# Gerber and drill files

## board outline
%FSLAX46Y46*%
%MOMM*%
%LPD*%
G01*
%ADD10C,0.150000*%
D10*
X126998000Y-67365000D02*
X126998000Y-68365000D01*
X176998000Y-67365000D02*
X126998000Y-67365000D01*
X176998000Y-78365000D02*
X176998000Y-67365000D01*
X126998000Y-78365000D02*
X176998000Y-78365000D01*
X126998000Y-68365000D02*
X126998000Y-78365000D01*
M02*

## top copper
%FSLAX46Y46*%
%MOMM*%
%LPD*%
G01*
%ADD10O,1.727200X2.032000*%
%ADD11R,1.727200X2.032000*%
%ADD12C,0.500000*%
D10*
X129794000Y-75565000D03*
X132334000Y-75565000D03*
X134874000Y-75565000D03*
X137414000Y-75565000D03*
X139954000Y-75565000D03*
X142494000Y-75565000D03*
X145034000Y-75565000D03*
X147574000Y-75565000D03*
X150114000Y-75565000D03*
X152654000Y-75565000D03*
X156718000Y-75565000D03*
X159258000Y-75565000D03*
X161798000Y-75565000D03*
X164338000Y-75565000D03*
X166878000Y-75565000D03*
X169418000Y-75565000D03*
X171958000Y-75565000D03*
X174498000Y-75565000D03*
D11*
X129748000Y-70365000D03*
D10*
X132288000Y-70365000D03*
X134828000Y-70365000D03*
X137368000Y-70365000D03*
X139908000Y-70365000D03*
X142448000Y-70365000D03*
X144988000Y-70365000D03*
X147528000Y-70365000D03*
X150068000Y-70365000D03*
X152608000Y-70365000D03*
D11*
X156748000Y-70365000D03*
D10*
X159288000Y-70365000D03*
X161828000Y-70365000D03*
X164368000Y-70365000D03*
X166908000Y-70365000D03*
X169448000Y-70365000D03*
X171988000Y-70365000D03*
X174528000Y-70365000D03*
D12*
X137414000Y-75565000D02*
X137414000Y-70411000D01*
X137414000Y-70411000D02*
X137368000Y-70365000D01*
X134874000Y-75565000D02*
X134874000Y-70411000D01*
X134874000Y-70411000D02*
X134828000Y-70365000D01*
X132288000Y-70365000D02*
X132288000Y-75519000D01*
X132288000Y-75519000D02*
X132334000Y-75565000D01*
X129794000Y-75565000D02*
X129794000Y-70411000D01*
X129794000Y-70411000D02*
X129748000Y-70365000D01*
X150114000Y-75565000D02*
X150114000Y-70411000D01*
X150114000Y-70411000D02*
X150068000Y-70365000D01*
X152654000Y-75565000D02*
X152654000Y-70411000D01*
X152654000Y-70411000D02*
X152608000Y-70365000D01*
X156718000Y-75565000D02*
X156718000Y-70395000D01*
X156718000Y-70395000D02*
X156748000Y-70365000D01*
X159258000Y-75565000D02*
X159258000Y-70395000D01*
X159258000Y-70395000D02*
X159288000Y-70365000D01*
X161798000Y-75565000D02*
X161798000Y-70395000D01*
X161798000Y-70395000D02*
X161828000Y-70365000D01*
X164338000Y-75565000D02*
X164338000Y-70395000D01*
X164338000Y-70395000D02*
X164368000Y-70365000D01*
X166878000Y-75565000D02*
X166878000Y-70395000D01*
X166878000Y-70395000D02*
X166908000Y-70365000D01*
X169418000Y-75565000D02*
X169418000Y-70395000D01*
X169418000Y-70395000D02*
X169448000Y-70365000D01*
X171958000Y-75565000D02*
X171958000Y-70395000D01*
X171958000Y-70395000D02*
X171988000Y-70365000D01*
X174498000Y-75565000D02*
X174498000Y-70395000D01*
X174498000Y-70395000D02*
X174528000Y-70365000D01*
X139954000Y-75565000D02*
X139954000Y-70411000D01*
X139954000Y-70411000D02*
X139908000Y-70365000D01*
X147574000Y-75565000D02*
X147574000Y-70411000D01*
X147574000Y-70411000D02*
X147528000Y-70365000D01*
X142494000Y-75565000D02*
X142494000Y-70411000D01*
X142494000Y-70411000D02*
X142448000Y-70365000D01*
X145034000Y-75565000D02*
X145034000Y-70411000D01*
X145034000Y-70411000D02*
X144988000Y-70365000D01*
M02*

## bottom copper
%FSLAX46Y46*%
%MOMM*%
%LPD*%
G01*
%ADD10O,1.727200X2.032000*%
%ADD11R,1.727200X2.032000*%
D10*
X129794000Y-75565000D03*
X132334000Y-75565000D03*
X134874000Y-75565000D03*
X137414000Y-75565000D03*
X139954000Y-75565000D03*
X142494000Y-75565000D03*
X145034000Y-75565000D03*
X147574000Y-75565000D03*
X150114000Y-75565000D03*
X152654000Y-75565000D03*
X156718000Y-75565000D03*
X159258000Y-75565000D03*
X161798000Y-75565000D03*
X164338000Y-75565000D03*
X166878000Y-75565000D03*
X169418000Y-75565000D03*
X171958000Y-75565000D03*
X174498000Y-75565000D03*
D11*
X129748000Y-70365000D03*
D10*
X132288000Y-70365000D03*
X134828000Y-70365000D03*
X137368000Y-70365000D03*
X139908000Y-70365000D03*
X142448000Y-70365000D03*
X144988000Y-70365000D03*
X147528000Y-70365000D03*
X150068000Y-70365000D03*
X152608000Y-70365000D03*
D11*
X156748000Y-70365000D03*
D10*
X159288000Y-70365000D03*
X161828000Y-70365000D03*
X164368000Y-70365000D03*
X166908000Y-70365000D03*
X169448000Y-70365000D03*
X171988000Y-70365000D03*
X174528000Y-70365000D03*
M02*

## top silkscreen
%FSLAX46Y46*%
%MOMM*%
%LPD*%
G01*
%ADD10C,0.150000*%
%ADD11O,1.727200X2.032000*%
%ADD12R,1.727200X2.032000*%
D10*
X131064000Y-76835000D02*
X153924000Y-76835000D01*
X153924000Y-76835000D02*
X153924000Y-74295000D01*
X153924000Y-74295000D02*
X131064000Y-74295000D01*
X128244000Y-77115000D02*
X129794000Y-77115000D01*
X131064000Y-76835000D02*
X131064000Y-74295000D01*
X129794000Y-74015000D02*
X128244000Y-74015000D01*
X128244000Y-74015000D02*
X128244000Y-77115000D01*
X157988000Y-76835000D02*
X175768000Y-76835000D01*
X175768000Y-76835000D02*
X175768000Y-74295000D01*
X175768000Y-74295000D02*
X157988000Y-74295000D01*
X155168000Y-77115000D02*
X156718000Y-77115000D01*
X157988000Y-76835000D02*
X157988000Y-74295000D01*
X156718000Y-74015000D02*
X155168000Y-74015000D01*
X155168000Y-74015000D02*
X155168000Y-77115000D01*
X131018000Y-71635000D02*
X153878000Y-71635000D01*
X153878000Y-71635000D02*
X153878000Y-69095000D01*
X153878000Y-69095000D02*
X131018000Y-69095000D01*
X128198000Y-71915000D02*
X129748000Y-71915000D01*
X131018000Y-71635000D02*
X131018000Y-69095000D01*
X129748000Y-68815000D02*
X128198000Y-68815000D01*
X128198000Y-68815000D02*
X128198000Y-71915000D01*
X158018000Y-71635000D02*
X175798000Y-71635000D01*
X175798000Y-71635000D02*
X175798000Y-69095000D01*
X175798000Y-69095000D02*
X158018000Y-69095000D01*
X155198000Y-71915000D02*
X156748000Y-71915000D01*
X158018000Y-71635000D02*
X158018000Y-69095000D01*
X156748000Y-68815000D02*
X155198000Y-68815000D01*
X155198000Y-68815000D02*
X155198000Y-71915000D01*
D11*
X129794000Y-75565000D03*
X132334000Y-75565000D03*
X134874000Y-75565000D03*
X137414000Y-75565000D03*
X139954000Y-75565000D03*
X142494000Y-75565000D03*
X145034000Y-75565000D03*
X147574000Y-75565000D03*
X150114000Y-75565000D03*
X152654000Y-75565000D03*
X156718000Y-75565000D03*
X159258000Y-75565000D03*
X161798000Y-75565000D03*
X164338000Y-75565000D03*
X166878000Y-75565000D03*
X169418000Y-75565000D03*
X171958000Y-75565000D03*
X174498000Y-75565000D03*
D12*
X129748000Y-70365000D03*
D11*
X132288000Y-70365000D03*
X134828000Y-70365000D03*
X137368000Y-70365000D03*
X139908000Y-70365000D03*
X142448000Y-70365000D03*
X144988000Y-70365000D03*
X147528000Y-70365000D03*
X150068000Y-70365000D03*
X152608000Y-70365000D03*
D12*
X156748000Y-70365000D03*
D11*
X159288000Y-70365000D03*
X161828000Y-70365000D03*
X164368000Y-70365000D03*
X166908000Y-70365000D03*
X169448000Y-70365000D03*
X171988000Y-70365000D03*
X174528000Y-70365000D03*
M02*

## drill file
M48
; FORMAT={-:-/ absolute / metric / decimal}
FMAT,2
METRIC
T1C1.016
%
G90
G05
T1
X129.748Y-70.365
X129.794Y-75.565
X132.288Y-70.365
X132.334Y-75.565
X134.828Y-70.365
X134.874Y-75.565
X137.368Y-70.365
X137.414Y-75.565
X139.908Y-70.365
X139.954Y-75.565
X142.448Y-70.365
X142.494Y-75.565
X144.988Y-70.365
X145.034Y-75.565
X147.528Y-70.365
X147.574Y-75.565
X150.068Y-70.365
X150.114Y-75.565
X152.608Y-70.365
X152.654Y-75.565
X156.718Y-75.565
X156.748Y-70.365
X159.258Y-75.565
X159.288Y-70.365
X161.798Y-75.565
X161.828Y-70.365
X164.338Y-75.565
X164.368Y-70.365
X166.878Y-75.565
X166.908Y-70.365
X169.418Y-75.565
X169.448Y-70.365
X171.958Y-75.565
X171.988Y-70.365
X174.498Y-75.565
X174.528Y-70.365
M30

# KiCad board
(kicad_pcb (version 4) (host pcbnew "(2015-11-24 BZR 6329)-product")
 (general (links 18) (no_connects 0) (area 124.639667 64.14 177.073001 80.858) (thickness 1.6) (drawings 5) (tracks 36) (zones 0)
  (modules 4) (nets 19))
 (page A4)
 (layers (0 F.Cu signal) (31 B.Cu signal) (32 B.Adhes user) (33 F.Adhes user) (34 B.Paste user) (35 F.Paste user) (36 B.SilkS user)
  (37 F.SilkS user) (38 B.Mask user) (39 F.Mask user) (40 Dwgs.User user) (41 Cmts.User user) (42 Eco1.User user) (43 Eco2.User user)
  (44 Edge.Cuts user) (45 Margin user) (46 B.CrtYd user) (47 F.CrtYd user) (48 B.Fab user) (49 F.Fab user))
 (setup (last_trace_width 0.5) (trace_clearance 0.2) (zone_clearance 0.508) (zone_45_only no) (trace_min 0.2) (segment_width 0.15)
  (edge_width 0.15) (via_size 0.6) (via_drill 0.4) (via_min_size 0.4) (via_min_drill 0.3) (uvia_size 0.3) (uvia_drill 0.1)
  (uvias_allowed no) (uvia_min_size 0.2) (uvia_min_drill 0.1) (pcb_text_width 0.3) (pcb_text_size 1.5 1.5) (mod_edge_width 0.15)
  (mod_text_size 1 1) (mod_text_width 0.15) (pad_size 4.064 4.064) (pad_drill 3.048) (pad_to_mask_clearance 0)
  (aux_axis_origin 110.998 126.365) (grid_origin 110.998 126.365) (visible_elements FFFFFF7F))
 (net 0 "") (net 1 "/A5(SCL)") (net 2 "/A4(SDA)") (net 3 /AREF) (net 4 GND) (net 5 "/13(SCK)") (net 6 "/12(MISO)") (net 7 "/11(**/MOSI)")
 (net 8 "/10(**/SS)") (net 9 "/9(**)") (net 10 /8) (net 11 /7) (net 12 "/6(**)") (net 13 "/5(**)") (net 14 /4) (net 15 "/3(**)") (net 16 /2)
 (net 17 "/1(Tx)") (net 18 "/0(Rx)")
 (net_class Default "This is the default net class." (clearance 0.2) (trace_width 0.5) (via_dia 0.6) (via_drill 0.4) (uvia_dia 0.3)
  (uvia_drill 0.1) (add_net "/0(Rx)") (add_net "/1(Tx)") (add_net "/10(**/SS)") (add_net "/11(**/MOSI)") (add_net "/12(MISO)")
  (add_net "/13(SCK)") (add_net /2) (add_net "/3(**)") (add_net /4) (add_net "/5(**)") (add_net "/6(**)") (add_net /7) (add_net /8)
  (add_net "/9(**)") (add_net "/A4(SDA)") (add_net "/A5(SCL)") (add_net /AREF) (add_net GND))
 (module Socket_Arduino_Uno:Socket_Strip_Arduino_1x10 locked (layer F.Cu) (at 129.794 75.565)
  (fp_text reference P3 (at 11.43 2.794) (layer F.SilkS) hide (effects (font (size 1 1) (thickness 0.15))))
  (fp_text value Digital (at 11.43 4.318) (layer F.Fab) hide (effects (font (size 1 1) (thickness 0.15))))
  (fp_line (start 1.27 1.27) (end 24.13 1.27) (layer F.SilkS) (width 0.15))
  (fp_line (start 24.13 1.27) (end 24.13 -1.27) (layer F.SilkS) (width 0.15))
  (fp_line (start 24.13 -1.27) (end 1.27 -1.27) (layer F.SilkS) (width 0.15))
  (fp_line (start -1.55 1.55) (end 0 1.55) (layer F.SilkS) (width 0.15))
  (fp_line (start 1.27 1.27) (end 1.27 -1.27) (layer F.SilkS) (width 0.15))
  (fp_line (start 0 -1.55) (end -1.55 -1.55) (layer F.SilkS) (width 0.15))
  (fp_line (start -1.55 -1.55) (end -1.55 1.55) (layer F.SilkS) (width 0.15))
  (pad 1 thru_hole oval (at 0 0) (size 1.7272 2.032) (drill 1.016) (layers *.Cu *.Mask F.SilkS) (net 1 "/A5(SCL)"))
  (pad 2 thru_hole oval (at 2.54 0) (size 1.7272 2.032) (drill 1.016) (layers *.Cu *.Mask F.SilkS) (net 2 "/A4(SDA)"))
  (pad 3 thru_hole oval (at 5.08 0) (size 1.7272 2.032) (drill 1.016) (layers *.Cu *.Mask F.SilkS) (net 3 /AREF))
  (pad 4 thru_hole oval (at 7.62 0) (size 1.7272 2.032) (drill 1.016) (layers *.Cu *.Mask F.SilkS) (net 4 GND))
  (pad 5 thru_hole oval (at 10.16 0) (size 1.7272 2.032) (drill 1.016) (layers *.Cu *.Mask F.SilkS) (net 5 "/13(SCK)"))
  (pad 6 thru_hole oval (at 12.7 0) (size 1.7272 2.032) (drill 1.016) (layers *.Cu *.Mask F.SilkS) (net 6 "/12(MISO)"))
  (pad 7 thru_hole oval (at 15.24 0) (size 1.7272 2.032) (drill 1.016) (layers *.Cu *.Mask F.SilkS) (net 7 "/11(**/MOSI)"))
  (pad 8 thru_hole oval (at 17.78 0) (size 1.7272 2.032) (drill 1.016) (layers *.Cu *.Mask F.SilkS) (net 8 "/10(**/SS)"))
  (pad 9 thru_hole oval (at 20.32 0) (size 1.7272 2.032) (drill 1.016) (layers *.Cu *.Mask F.SilkS) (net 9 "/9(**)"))
  (pad 10 thru_hole oval (at 22.86 0) (size 1.7272 2.032) (drill 1.016) (layers *.Cu *.Mask F.SilkS) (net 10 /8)))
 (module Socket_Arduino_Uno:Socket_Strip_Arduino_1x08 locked (layer F.Cu) (at 156.718 75.565)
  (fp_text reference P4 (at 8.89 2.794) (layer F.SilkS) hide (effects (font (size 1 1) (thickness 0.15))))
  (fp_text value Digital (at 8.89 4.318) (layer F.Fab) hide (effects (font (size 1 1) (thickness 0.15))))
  (fp_line (start 1.27 1.27) (end 19.05 1.27) (layer F.SilkS) (width 0.15))
  (fp_line (start 19.05 1.27) (end 19.05 -1.27) (layer F.SilkS) (width 0.15))
  (fp_line (start 19.05 -1.27) (end 1.27 -1.27) (layer F.SilkS) (width 0.15))
  (fp_line (start -1.55 1.55) (end 0 1.55) (layer F.SilkS) (width 0.15))
  (fp_line (start 1.27 1.27) (end 1.27 -1.27) (layer F.SilkS) (width 0.15))
  (fp_line (start 0 -1.55) (end -1.55 -1.55) (layer F.SilkS) (width 0.15))
  (fp_line (start -1.55 -1.55) (end -1.55 1.55) (layer F.SilkS) (width 0.15))
  (pad 1 thru_hole oval (at 0 0) (size 1.7272 2.032) (drill 1.016) (layers *.Cu *.Mask F.SilkS) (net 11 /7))
  (pad 2 thru_hole oval (at 2.54 0) (size 1.7272 2.032) (drill 1.016) (layers *.Cu *.Mask F.SilkS) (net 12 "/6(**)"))
  (pad 3 thru_hole oval (at 5.08 0) (size 1.7272 2.032) (drill 1.016) (layers *.Cu *.Mask F.SilkS) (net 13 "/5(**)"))
  (pad 4 thru_hole oval (at 7.62 0) (size 1.7272 2.032) (drill 1.016) (layers *.Cu *.Mask F.SilkS) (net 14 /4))
  (pad 5 thru_hole oval (at 10.16 0) (size 1.7272 2.032) (drill 1.016) (layers *.Cu *.Mask F.SilkS) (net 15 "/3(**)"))
  (pad 6 thru_hole oval (at 12.7 0) (size 1.7272 2.032) (drill 1.016) (layers *.Cu *.Mask F.SilkS) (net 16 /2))
  (pad 7 thru_hole oval (at 15.24 0) (size 1.7272 2.032) (drill 1.016) (layers *.Cu *.Mask F.SilkS) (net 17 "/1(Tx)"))
  (pad 8 thru_hole oval (at 17.78 0) (size 1.7272 2.032) (drill 1.016) (layers *.Cu *.Mask F.SilkS) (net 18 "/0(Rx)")))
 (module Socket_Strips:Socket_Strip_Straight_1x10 (layer F.Cu) (at 129.748 70.365)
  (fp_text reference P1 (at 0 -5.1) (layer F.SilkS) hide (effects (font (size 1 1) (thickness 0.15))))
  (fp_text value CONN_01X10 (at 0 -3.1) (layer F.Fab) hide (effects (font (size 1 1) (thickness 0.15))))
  (fp_line (start 1.27 1.27) (end 24.13 1.27) (layer F.SilkS) (width 0.15))
  (fp_line (start 24.13 1.27) (end 24.13 -1.27) (layer F.SilkS) (width 0.15))
  (fp_line (start 24.13 -1.27) (end 1.27 -1.27) (layer F.SilkS) (width 0.15))
  (fp_line (start -1.55 1.55) (end 0 1.55) (layer F.SilkS) (width 0.15))
  (fp_line (start 1.27 1.27) (end 1.27 -1.27) (layer F.SilkS) (width 0.15))
  (fp_line (start 0 -1.55) (end -1.55 -1.55) (layer F.SilkS) (width 0.15))
  (fp_line (start -1.55 -1.55) (end -1.55 1.55) (layer F.SilkS) (width 0.15))
  (pad 1 thru_hole rect (at 0 0) (size 1.7272 2.032) (drill 1.016) (layers *.Cu *.Mask F.SilkS) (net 1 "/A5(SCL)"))
  (pad 2 thru_hole oval (at 2.54 0) (size 1.7272 2.032) (drill 1.016) (layers *.Cu *.Mask F.SilkS) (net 2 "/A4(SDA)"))
  (pad 3 thru_hole oval (at 5.08 0) (size 1.7272 2.032) (drill 1.016) (layers *.Cu *.Mask F.SilkS) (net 3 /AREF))
  (pad 4 thru_hole oval (at 7.62 0) (size 1.7272 2.032) (drill 1.016) (layers *.Cu *.Mask F.SilkS) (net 4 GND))
  (pad 5 thru_hole oval (at 10.16 0) (size 1.7272 2.032) (drill 1.016) (layers *.Cu *.Mask F.SilkS) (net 5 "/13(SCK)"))
  (pad 6 thru_hole oval (at 12.7 0) (size 1.7272 2.032) (drill 1.016) (layers *.Cu *.Mask F.SilkS) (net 6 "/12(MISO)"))
  (pad 7 thru_hole oval (at 15.24 0) (size 1.7272 2.032) (drill 1.016) (layers *.Cu *.Mask F.SilkS) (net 7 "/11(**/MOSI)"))
  (pad 8 thru_hole oval (at 17.78 0) (size 1.7272 2.032) (drill 1.016) (layers *.Cu *.Mask F.SilkS) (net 8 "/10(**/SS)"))
  (pad 9 thru_hole oval (at 20.32 0) (size 1.7272 2.032) (drill 1.016) (layers *.Cu *.Mask F.SilkS) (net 9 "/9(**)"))
  (pad 10 thru_hole oval (at 22.86 0) (size 1.7272 2.032) (drill 1.016) (layers *.Cu *.Mask F.SilkS) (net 10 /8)))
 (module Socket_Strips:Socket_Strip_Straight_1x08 (layer F.Cu) (at 156.748 70.365)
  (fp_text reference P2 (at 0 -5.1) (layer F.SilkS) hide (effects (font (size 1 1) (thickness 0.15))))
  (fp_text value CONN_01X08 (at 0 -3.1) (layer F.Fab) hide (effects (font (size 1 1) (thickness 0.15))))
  (fp_line (start 1.27 1.27) (end 19.05 1.27) (layer F.SilkS) (width 0.15))
  (fp_line (start 19.05 1.27) (end 19.05 -1.27) (layer F.SilkS) (width 0.15))
  (fp_line (start 19.05 -1.27) (end 1.27 -1.27) (layer F.SilkS) (width 0.15))
  (fp_line (start -1.55 1.55) (end 0 1.55) (layer F.SilkS) (width 0.15))
  (fp_line (start 1.27 1.27) (end 1.27 -1.27) (layer F.SilkS) (width 0.15))
  (fp_line (start 0 -1.55) (end -1.55 -1.55) (layer F.SilkS) (width 0.15))
  (fp_line (start -1.55 -1.55) (end -1.55 1.55) (layer F.SilkS) (width 0.15))
  (pad 1 thru_hole rect (at 0 0) (size 1.7272 2.032) (drill 1.016) (layers *.Cu *.Mask F.SilkS) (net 11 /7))
  (pad 2 thru_hole oval (at 2.54 0) (size 1.7272 2.032) (drill 1.016) (layers *.Cu *.Mask F.SilkS) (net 12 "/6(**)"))
  (pad 3 thru_hole oval (at 5.08 0) (size 1.7272 2.032) (drill 1.016) (layers *.Cu *.Mask F.SilkS) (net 13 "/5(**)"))
  (pad 4 thru_hole oval (at 7.62 0) (size 1.7272 2.032) (drill 1.016) (layers *.Cu *.Mask F.SilkS) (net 14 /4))
  (pad 5 thru_hole oval (at 10.16 0) (size 1.7272 2.032) (drill 1.016) (layers *.Cu *.Mask F.SilkS) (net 15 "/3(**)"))
  (pad 6 thru_hole oval (at 12.7 0) (size 1.7272 2.032) (drill 1.016) (layers *.Cu *.Mask F.SilkS) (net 16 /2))
  (pad 7 thru_hole oval (at 15.24 0) (size 1.7272 2.032) (drill 1.016) (layers *.Cu *.Mask F.SilkS) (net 17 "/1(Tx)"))
  (pad 8 thru_hole oval (at 17.78 0) (size 1.7272 2.032) (drill 1.016) (layers *.Cu *.Mask F.SilkS) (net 18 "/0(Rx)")))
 (gr_line (start 126.998 67.365) (end 126.998 68.365) (angle 90) (layer Edge.Cuts) (width 0.15))
 (gr_line (start 176.998 67.365) (end 126.998 67.365) (angle 90) (layer Edge.Cuts) (width 0.15))
 (gr_line (start 176.998 78.365) (end 176.998 67.365) (angle 90) (layer Edge.Cuts) (width 0.15))
 (gr_line (start 126.998 78.365) (end 176.998 78.365) (angle 90) (layer Edge.Cuts) (width 0.15))
 (gr_line (start 126.998 68.365) (end 126.998 78.365) (angle 90) (layer Edge.Cuts) (width 0.15))
 (segment (start 137.414 75.565) (end 137.414 70.411) (width 0.5) (layer F.Cu) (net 4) (status C00000))
 (segment (start 137.414 70.411) (end 137.368 70.365) (width 0.5) (layer F.Cu) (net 4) (status C00000))
 (segment (start 134.874 75.565) (end 134.874 70.411) (width 0.5) (layer F.Cu) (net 3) (status C00000))
 (segment (start 134.874 70.411) (end 134.828 70.365) (width 0.5) (layer F.Cu) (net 3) (status C00000))
 (segment (start 132.288 70.365) (end 132.288 75.519) (width 0.5) (layer F.Cu) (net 2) (status C00000))
 (segment (start 132.288 75.519) (end 132.334 75.565) (width 0.5) (layer F.Cu) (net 2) (status C00000))
 (segment (start 129.794 75.565) (end 129.794 70.411) (width 0.5) (layer F.Cu) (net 1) (status C00000))
 (segment (start 129.794 70.411) (end 129.748 70.365) (width 0.5) (layer F.Cu) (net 1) (status C00000))
 (segment (start 150.114 75.565) (end 150.114 70.411) (width 0.5) (layer F.Cu) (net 9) (status C00000))
 (segment (start 150.114 70.411) (end 150.068 70.365) (width 0.5) (layer F.Cu) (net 9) (status C00000))
 (segment (start 152.654 75.565) (end 152.654 70.411) (width 0.5) (layer F.Cu) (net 10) (status C00000))
 (segment (start 152.654 70.411) (end 152.608 70.365) (width 0.5) (layer F.Cu) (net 10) (status C00000))
 (segment (start 156.718 75.565) (end 156.718 70.395) (width 0.5) (layer F.Cu) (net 11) (status C00000))
 (segment (start 156.718 70.395) (end 156.748 70.365) (width 0.5) (layer F.Cu) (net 11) (status C00000))
 (segment (start 159.258 75.565) (end 159.258 70.395) (width 0.5) (layer F.Cu) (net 12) (status C00000))
 (segment (start 159.258 70.395) (end 159.288 70.365) (width 0.5) (layer F.Cu) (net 12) (status C00000))
 (segment (start 161.798 75.565) (end 161.798 70.395) (width 0.5) (layer F.Cu) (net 13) (status C00000))
 (segment (start 161.798 70.395) (end 161.828 70.365) (width 0.5) (layer F.Cu) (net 13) (status C00000))
 (segment (start 164.338 75.565) (end 164.338 70.395) (width 0.5) (layer F.Cu) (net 14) (status C00000))
 (segment (start 164.338 70.395) (end 164.368 70.365) (width 0.5) (layer F.Cu) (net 14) (status C00000))
 (segment (start 166.878 75.565) (end 166.878 70.395) (width 0.5) (layer F.Cu) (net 15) (status C00000))
 (segment (start 166.878 70.395) (end 166.908 70.365) (width 0.5) (layer F.Cu) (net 15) (status C00000))
 (segment (start 169.418 75.565) (end 169.418 70.395) (width 0.5) (layer F.Cu) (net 16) (status C00000))
 (segment (start 169.418 70.395) (end 169.448 70.365) (width 0.5) (layer F.Cu) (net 16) (status C00000))
 (segment (start 171.958 75.565) (end 171.958 70.395) (width 0.5) (layer F.Cu) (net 17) (status C00000))
 (segment (start 171.958 70.395) (end 171.988 70.365) (width 0.5) (layer F.Cu) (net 17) (status C00000))
 (segment (start 174.498 75.565) (end 174.498 70.395) (width 0.5) (layer F.Cu) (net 18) (status C00000))
 (segment (start 174.498 70.395) (end 174.528 70.365) (width 0.5) (layer F.Cu) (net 18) (status C00000))
 (segment (start 139.954 75.565) (end 139.954 70.411) (width 0.5) (layer F.Cu) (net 5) (status C00000))
 (segment (start 139.954 70.411) (end 139.908 70.365) (width 0.5) (layer F.Cu) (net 5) (status C00000))
 (segment (start 147.574 75.565) (end 147.574 70.411) (width 0.5) (layer F.Cu) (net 8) (status C00000))
 (segment (start 147.574 70.411) (end 147.528 70.365) (width 0.5) (layer F.Cu) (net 8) (status C00000))
 (segment (start 142.494 75.565) (end 142.494 70.411) (width 0.5) (layer F.Cu) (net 6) (status C00000))
 (segment (start 142.494 70.411) (end 142.448 70.365) (width 0.5) (layer F.Cu) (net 6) (status C00000))
 (segment (start 145.034 75.565) (end 145.034 70.411) (width 0.5) (layer F.Cu) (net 7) (status C00000))
 (segment (start 145.034 70.411) (end 144.988 70.365) (width 0.5) (layer F.Cu) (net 7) (status C00000)))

